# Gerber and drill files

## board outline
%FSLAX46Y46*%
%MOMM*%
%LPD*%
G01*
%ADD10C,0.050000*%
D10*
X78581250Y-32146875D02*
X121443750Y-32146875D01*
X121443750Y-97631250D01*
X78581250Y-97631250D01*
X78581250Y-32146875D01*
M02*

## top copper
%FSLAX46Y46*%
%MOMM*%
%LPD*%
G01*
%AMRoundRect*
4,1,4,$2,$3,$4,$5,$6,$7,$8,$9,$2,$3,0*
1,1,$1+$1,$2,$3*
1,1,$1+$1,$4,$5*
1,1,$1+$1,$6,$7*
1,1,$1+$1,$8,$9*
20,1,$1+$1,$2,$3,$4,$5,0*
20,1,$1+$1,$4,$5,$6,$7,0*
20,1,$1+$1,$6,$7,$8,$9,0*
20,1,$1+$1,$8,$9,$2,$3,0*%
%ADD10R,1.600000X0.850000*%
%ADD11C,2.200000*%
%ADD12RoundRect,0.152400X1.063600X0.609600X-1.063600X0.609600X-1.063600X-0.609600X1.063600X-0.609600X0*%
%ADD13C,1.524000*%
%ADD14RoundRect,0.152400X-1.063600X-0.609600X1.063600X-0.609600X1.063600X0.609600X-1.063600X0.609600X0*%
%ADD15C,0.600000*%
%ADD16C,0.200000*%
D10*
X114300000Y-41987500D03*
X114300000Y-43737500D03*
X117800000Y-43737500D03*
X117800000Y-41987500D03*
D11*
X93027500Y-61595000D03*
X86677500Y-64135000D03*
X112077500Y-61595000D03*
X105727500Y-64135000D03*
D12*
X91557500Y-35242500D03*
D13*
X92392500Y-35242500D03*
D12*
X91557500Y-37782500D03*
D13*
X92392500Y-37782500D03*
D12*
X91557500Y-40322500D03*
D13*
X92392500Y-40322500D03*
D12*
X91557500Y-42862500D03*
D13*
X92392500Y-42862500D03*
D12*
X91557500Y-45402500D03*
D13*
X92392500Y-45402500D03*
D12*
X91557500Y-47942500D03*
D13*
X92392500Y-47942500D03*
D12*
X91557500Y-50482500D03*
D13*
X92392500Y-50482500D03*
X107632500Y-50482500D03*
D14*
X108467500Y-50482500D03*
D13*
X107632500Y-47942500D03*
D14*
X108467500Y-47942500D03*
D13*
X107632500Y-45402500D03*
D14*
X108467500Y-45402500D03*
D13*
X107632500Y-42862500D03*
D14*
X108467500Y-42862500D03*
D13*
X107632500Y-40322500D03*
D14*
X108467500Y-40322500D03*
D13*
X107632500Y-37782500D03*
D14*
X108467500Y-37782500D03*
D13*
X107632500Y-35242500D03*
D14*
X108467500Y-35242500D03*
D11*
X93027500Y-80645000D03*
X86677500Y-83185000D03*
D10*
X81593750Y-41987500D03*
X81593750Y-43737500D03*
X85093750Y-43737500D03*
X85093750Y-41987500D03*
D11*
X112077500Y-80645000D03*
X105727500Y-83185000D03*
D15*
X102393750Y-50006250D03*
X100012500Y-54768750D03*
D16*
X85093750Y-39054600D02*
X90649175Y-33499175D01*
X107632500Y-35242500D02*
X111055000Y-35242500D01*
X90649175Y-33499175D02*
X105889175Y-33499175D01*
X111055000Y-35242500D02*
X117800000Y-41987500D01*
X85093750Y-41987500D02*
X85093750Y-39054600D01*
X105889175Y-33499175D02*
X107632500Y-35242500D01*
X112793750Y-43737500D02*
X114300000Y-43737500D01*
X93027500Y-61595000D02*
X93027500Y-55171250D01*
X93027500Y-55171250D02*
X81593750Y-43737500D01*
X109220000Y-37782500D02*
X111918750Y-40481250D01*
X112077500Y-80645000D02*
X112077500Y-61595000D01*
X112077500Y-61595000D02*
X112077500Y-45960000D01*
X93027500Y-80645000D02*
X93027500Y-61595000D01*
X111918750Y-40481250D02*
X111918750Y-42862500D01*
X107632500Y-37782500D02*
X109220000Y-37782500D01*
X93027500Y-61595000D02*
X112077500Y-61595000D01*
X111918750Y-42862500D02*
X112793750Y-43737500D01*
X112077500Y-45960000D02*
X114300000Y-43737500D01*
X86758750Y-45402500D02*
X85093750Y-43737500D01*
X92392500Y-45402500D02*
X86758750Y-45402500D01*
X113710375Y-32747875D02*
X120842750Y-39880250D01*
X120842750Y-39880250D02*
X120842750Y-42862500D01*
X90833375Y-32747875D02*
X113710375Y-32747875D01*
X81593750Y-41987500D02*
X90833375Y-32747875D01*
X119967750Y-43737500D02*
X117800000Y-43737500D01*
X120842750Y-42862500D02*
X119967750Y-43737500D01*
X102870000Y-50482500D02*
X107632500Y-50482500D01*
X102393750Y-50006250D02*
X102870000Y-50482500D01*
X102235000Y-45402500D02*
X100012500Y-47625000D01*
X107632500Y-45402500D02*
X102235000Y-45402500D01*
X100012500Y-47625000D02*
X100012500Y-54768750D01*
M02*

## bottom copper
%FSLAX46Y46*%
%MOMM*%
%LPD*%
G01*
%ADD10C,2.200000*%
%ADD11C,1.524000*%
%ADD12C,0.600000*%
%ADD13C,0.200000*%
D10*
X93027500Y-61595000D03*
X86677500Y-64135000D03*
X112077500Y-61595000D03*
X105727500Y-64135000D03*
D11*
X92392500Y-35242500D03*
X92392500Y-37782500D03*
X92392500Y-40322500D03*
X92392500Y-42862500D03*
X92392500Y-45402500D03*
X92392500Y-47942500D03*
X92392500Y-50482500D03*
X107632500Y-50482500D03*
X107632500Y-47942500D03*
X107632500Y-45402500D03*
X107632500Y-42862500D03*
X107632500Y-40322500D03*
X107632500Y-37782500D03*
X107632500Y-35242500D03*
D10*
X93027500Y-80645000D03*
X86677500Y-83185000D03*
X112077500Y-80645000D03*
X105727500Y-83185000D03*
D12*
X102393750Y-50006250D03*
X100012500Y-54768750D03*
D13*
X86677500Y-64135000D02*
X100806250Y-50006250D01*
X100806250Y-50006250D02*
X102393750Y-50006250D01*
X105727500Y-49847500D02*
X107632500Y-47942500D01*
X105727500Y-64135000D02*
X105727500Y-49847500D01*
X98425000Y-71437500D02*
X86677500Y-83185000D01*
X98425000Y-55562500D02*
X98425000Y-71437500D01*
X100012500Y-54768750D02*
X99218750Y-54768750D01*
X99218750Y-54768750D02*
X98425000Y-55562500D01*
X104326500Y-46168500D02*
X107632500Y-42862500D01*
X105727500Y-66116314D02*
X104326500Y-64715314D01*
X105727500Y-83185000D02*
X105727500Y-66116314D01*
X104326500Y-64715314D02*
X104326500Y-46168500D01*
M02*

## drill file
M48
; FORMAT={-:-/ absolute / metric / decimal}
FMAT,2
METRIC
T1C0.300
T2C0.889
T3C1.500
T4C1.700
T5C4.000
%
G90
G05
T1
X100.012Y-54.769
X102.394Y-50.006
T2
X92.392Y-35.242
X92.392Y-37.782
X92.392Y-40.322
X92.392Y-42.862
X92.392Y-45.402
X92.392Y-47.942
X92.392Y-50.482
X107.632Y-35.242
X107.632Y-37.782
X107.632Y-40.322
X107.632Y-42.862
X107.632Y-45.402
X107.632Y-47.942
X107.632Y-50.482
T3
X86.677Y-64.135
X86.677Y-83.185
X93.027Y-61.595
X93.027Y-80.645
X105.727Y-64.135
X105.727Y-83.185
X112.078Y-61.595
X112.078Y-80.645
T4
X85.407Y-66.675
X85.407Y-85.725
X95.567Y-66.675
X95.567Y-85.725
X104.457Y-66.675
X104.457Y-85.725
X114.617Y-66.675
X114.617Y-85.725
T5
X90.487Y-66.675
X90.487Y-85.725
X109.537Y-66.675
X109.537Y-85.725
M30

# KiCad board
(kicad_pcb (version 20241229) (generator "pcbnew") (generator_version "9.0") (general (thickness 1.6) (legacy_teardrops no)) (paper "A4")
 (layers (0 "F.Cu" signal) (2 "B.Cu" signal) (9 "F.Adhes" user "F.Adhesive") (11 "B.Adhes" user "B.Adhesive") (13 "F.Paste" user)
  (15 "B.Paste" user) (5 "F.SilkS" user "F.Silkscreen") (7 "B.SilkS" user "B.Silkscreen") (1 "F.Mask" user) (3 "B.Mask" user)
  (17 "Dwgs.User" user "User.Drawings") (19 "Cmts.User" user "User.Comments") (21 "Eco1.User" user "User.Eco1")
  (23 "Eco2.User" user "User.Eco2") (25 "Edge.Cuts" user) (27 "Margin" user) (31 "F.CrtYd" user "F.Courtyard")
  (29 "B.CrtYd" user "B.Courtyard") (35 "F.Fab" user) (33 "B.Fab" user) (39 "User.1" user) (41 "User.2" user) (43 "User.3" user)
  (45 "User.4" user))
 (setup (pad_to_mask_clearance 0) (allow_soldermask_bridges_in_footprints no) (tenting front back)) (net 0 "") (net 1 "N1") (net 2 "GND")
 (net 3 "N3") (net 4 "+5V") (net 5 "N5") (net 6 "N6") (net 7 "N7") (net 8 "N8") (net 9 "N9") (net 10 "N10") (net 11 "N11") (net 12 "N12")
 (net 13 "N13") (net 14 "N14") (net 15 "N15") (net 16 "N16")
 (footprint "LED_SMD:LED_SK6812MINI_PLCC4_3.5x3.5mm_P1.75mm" (layer "F.Cu") (at 116.05 42.8625)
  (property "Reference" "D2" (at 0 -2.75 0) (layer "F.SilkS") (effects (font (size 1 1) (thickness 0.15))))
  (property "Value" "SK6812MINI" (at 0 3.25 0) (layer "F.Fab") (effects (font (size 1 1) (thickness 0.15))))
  (pad "1" smd rect (at -1.75 -0.875) (size 1.6 0.85) (layers "F.Cu" "F.Mask" "F.Paste") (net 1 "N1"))
  (pad "2" smd rect (at -1.75 0.875) (size 1.6 0.85) (layers "F.Cu" "F.Mask" "F.Paste") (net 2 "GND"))
  (pad "3" smd rect (at 1.75 0.875) (size 1.6 0.85) (layers "F.Cu" "F.Mask" "F.Paste") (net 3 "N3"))
  (pad "4" smd rect (at 1.75 -0.875) (size 1.6 0.85) (layers "F.Cu" "F.Mask" "F.Paste") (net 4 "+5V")))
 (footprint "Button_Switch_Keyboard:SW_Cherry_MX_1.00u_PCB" (layer "F.Cu") (at 93.0275 61.595)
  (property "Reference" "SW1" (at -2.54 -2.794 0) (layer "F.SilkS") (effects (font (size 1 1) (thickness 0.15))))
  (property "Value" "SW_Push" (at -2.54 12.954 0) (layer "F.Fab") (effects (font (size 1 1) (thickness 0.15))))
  (pad "" np_thru_hole circle (at -7.62 5.08) (size 1.7 1.7) (drill 1.7) (layers "*.Cu" "*.Mask"))
  (pad "" np_thru_hole circle (at -2.54 5.08) (size 4 4) (drill 4) (layers "*.Cu" "*.Mask"))
  (pad "" np_thru_hole circle (at 2.54 5.08) (size 1.7 1.7) (drill 1.7) (layers "*.Cu" "*.Mask"))
  (pad "1" thru_hole circle (at 0 0) (size 2.2 2.2) (drill 1.5) (layers "*.Cu" "*.Mask") (remove_unused_layers no) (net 2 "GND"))
  (pad "2" thru_hole circle (at -6.35 2.54) (size 2.2 2.2) (drill 1.5) (layers "*.Cu" "*.Mask") (remove_unused_layers no) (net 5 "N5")))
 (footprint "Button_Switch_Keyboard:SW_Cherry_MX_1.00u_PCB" (layer "F.Cu") (at 112.0775 61.595)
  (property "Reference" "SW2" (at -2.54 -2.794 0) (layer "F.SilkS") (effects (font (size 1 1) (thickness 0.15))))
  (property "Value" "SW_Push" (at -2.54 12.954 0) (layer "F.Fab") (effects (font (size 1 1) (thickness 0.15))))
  (pad "" np_thru_hole circle (at -7.62 5.08) (size 1.7 1.7) (drill 1.7) (layers "*.Cu" "*.Mask"))
  (pad "" np_thru_hole circle (at -2.54 5.08) (size 4 4) (drill 4) (layers "*.Cu" "*.Mask"))
  (pad "" np_thru_hole circle (at 2.54 5.08) (size 1.7 1.7) (drill 1.7) (layers "*.Cu" "*.Mask"))
  (pad "1" thru_hole circle (at 0 0) (size 2.2 2.2) (drill 1.5) (layers "*.Cu" "*.Mask") (remove_unused_layers no) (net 2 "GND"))
  (pad "2" thru_hole circle (at -6.35 2.54) (size 2.2 2.2) (drill 1.5) (layers "*.Cu" "*.Mask") (remove_unused_layers no) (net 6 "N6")))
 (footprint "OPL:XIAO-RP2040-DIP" (layer "F.Cu") (at 100.0125 42.8625)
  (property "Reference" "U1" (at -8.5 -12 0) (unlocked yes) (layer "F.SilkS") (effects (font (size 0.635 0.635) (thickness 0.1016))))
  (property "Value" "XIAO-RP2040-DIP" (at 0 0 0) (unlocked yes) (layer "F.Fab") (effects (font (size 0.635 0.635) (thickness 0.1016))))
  (pad "1" smd roundrect (at -8.455 -7.62 180) (size 2.432 1.524) (layers "F.Cu" "F.Mask") (roundrect_rratio 0.1) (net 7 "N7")
   (thermal_bridge_angle 45))
  (pad "1" thru_hole circle (at -7.62 -7.62 180) (size 1.524 1.524) (drill 0.889) (layers "*.Cu" "*.Mask") (remove_unused_layers no)
   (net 7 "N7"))
  (pad "2" smd roundrect (at -8.455 -5.08 180) (size 2.432 1.524) (layers "F.Cu" "F.Mask") (roundrect_rratio 0.1) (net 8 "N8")
   (thermal_bridge_angle 45))
  (pad "2" thru_hole circle (at -7.62 -5.08 180) (size 1.524 1.524) (drill 0.889) (layers "*.Cu" "*.Mask") (remove_unused_layers no)
   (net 8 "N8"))
  (pad "3" smd roundrect (at -8.455 -2.54 180) (size 2.432 1.524) (layers "F.Cu" "F.Mask") (roundrect_rratio 0.1) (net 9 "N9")
   (thermal_bridge_angle 45))
  (pad "3" thru_hole circle (at -7.62 -2.54 180) (size 1.524 1.524) (drill 0.889) (layers "*.Cu" "*.Mask") (remove_unused_layers no)
   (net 9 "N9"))
  (pad "4" smd roundrect (at -8.455 0 180) (size 2.432 1.524) (layers "F.Cu" "F.Mask") (roundrect_rratio 0.1) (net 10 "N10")
   (thermal_bridge_angle 45))
  (pad "4" thru_hole circle (at -7.62 0 180) (size 1.524 1.524) (drill 0.889) (layers "*.Cu" "*.Mask") (remove_unused_layers no)
   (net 10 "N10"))
  (pad "5" smd roundrect (at -8.455 2.54 180) (size 2.432 1.524) (layers "F.Cu" "F.Mask") (roundrect_rratio 0.1) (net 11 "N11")
   (thermal_bridge_angle 45))
  (pad "5" thru_hole circle (at -7.62 2.54 180) (size 1.524 1.524) (drill 0.889) (layers "*.Cu" "*.Mask") (remove_unused_layers no)
   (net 11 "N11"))
  (pad "6" smd roundrect (at -8.455 5.08 180) (size 2.432 1.524) (layers "F.Cu" "F.Mask") (roundrect_rratio 0.1) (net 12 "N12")
   (thermal_bridge_angle 45))
  (pad "6" thru_hole circle (at -7.62 5.08 180) (size 1.524 1.524) (drill 0.889) (layers "*.Cu" "*.Mask") (remove_unused_layers no)
   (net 12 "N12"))
  (pad "7" smd roundrect (at -8.455 7.62 180) (size 2.432 1.524) (layers "F.Cu" "F.Mask") (roundrect_rratio 0.1) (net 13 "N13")
   (thermal_bridge_angle 45))
  (pad "7" thru_hole circle (at -7.62 7.62 180) (size 1.524 1.524) (drill 0.889) (layers "*.Cu" "*.Mask") (remove_unused_layers no)
   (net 13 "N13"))
  (pad "8" thru_hole circle (at 7.62 7.62) (size 1.524 1.524) (drill 0.889) (layers "*.Cu" "*.Mask") (remove_unused_layers no) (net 5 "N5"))
  (pad "8" smd roundrect (at 8.455 7.62) (size 2.432 1.524) (layers "F.Cu" "F.Mask") (roundrect_rratio 0.1) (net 5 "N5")
   (thermal_bridge_angle 45))
  (pad "9" thru_hole circle (at 7.62 5.08) (size 1.524 1.524) (drill 0.889) (layers "*.Cu" "*.Mask") (remove_unused_layers no) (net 6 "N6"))
  (pad "9" smd roundrect (at 8.455 5.08) (size 2.432 1.524) (layers "F.Cu" "F.Mask") (roundrect_rratio 0.1) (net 6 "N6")
   (thermal_bridge_angle 45))
  (pad "10" thru_hole circle (at 7.62 2.54) (size 1.524 1.524) (drill 0.889) (layers "*.Cu" "*.Mask") (remove_unused_layers no)
   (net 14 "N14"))
  (pad "10" smd roundrect (at 8.455 2.54) (size 2.432 1.524) (layers "F.Cu" "F.Mask") (roundrect_rratio 0.1) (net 14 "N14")
   (thermal_bridge_angle 45))
  (pad "11" thru_hole circle (at 7.62 0) (size 1.524 1.524) (drill 0.889) (layers "*.Cu" "*.Mask") (remove_unused_layers no) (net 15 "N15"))
  (pad "11" smd roundrect (at 8.455 0) (size 2.432 1.524) (layers "F.Cu" "F.Mask") (roundrect_rratio 0.1) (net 15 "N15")
   (thermal_bridge_angle 45))
  (pad "12" thru_hole circle (at 7.62 -2.54) (size 1.524 1.524) (drill 0.889) (layers "*.Cu" "*.Mask") (remove_unused_layers no)
   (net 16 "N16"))
  (pad "12" smd roundrect (at 8.455 -2.54) (size 2.432 1.524) (layers "F.Cu" "F.Mask") (roundrect_rratio 0.1) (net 16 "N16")
   (thermal_bridge_angle 45))
  (pad "13" thru_hole circle (at 7.62 -5.08) (size 1.524 1.524) (drill 0.889) (layers "*.Cu" "*.Mask") (remove_unused_layers no)
   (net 2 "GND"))
  (pad "13" smd roundrect (at 8.455 -5.08) (size 2.432 1.524) (layers "F.Cu" "F.Mask") (roundrect_rratio 0.1) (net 2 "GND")
   (thermal_bridge_angle 45))
  (pad "14" thru_hole circle (at 7.62 -7.62) (size 1.524 1.524) (drill 0.889) (layers "*.Cu" "*.Mask") (remove_unused_layers no)
   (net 4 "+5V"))
  (pad "14" smd roundrect (at 8.455 -7.62) (size 2.432 1.524) (layers "F.Cu" "F.Mask") (roundrect_rratio 0.1) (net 4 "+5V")
   (thermal_bridge_angle 45)))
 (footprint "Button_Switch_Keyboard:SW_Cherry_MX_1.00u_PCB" (layer "F.Cu") (at 93.0275 80.645)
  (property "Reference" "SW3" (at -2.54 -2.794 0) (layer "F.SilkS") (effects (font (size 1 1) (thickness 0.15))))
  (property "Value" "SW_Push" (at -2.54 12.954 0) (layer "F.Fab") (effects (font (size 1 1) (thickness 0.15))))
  (pad "" np_thru_hole circle (at -7.62 5.08) (size 1.7 1.7) (drill 1.7) (layers "*.Cu" "*.Mask"))
  (pad "" np_thru_hole circle (at -2.54 5.08) (size 4 4) (drill 4) (layers "*.Cu" "*.Mask"))
  (pad "" np_thru_hole circle (at 2.54 5.08) (size 1.7 1.7) (drill 1.7) (layers "*.Cu" "*.Mask"))
  (pad "1" thru_hole circle (at 0 0) (size 2.2 2.2) (drill 1.5) (layers "*.Cu" "*.Mask") (remove_unused_layers no) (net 2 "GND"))
  (pad "2" thru_hole circle (at -6.35 2.54) (size 2.2 2.2) (drill 1.5) (layers "*.Cu" "*.Mask") (remove_unused_layers no) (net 14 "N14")))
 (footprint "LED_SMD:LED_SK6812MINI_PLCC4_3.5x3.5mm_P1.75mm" (layer "F.Cu") (at 83.34375 42.8625)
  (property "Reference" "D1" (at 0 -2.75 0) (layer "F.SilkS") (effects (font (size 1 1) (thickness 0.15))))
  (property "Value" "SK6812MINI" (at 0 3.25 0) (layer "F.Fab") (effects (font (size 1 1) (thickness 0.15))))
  (pad "1" smd rect (at -1.75 -0.875) (size 1.6 0.85) (layers "F.Cu" "F.Mask" "F.Paste") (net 3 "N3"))
  (pad "2" smd rect (at -1.75 0.875) (size 1.6 0.85) (layers "F.Cu" "F.Mask" "F.Paste") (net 2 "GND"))
  (pad "3" smd rect (at 1.75 0.875) (size 1.6 0.85) (layers "F.Cu" "F.Mask" "F.Paste") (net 11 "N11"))
  (pad "4" smd rect (at 1.75 -0.875) (size 1.6 0.85) (layers "F.Cu" "F.Mask" "F.Paste") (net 4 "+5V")))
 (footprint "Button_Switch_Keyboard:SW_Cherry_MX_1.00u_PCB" (layer "F.Cu") (at 112.0775 80.645)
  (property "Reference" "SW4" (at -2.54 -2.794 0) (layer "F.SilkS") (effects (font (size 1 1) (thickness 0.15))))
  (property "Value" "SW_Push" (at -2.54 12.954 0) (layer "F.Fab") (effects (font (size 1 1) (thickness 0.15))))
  (pad "" np_thru_hole circle (at -7.62 5.08) (size 1.7 1.7) (drill 1.7) (layers "*.Cu" "*.Mask"))
  (pad "" np_thru_hole circle (at -2.54 5.08) (size 4 4) (drill 4) (layers "*.Cu" "*.Mask"))
  (pad "" np_thru_hole circle (at 2.54 5.08) (size 1.7 1.7) (drill 1.7) (layers "*.Cu" "*.Mask"))
  (pad "1" thru_hole circle (at 0 0) (size 2.2 2.2) (drill 1.5) (layers "*.Cu" "*.Mask") (remove_unused_layers no) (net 2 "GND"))
  (pad "2" thru_hole circle (at -6.35 2.54) (size 2.2 2.2) (drill 1.5) (layers "*.Cu" "*.Mask") (remove_unused_layers no) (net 15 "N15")))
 (gr_rect (start 78.58125 32.146875) (end 121.44375 97.63125) (stroke (width 0.05) (type solid)) (fill no) (layer "Edge.Cuts"))
 (segment (start 85.09375 39.0546) (end 90.649175 33.499175) (width 0.2) (layer "F.Cu") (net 4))
 (segment (start 107.6325 35.2425) (end 111.055 35.2425) (width 0.2) (layer "F.Cu") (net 4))
 (segment (start 90.649175 33.499175) (end 105.889175 33.499175) (width 0.2) (layer "F.Cu") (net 4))
 (segment (start 111.055 35.2425) (end 117.8 41.9875) (width 0.2) (layer "F.Cu") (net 4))
 (segment (start 85.09375 41.9875) (end 85.09375 39.0546) (width 0.2) (layer "F.Cu") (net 4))
 (segment (start 105.889175 33.499175) (end 107.6325 35.2425) (width 0.2) (layer "F.Cu") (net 4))
 (segment (start 112.79375 43.7375) (end 114.3 43.7375) (width 0.2) (layer "F.Cu") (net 2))
 (segment (start 93.0275 61.595) (end 93.0275 55.17125) (width 0.2) (layer "F.Cu") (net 2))
 (segment (start 93.0275 55.17125) (end 81.59375 43.7375) (width 0.2) (layer "F.Cu") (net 2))
 (segment (start 109.22 37.7825) (end 111.91875 40.48125) (width 0.2) (layer "F.Cu") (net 2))
 (segment (start 112.0775 80.645) (end 112.0775 61.595) (width 0.2) (layer "F.Cu") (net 2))
 (segment (start 112.0775 61.595) (end 112.0775 45.96) (width 0.2) (layer "F.Cu") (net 2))
 (segment (start 93.0275 80.645) (end 93.0275 61.595) (width 0.2) (layer "F.Cu") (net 2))
 (segment (start 111.91875 40.48125) (end 111.91875 42.8625) (width 0.2) (layer "F.Cu") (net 2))
 (segment (start 107.6325 37.7825) (end 109.22 37.7825) (width 0.2) (layer "F.Cu") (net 2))
 (segment (start 93.0275 61.595) (end 112.0775 61.595) (width 0.2) (layer "F.Cu") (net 2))
 (segment (start 111.91875 42.8625) (end 112.79375 43.7375) (width 0.2) (layer "F.Cu") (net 2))
 (segment (start 112.0775 45.96) (end 114.3 43.7375) (width 0.2) (layer "F.Cu") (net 2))
 (segment (start 86.75875 45.4025) (end 85.09375 43.7375) (width 0.2) (layer "F.Cu") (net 11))
 (segment (start 92.3925 45.4025) (end 86.75875 45.4025) (width 0.2) (layer "F.Cu") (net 11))
 (segment (start 113.710375 32.747875) (end 120.84275 39.88025) (width 0.2) (layer "F.Cu") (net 3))
 (segment (start 120.84275 39.88025) (end 120.84275 42.8625) (width 0.2) (layer "F.Cu") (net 3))
 (segment (start 90.833375 32.747875) (end 113.710375 32.747875) (width 0.2) (layer "F.Cu") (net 3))
 (segment (start 81.59375 41.9875) (end 90.833375 32.747875) (width 0.2) (layer "F.Cu") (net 3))
 (segment (start 119.96775 43.7375) (end 117.8 43.7375) (width 0.2) (layer "F.Cu") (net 3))
 (segment (start 120.84275 42.8625) (end 119.96775 43.7375) (width 0.2) (layer "F.Cu") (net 3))
 (segment (start 102.87 50.4825) (end 107.6325 50.4825) (width 0.2) (layer "F.Cu") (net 5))
 (segment (start 102.39375 50.00625) (end 102.87 50.4825) (width 0.2) (layer "F.Cu") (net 5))
 (via (at 102.39375 50.00625) (size 0.6) (drill 0.3) (layers "F.Cu" "B.Cu") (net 5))
 (segment (start 86.6775 64.135) (end 100.80625 50.00625) (width 0.2) (layer "B.Cu") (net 5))
 (segment (start 100.80625 50.00625) (end 102.39375 50.00625) (width 0.2) (layer "B.Cu") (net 5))
 (segment (start 105.7275 49.8475) (end 107.6325 47.9425) (width 0.2) (layer "B.Cu") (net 6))
 (segment (start 105.7275 64.135) (end 105.7275 49.8475) (width 0.2) (layer "B.Cu") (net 6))
 (segment (start 102.235 45.4025) (end 100.0125 47.625) (width 0.2) (layer "F.Cu") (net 14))
 (segment (start 107.6325 45.4025) (end 102.235 45.4025) (width 0.2) (layer "F.Cu") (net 14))
 (segment (start 100.0125 47.625) (end 100.0125 54.76875) (width 0.2) (layer "F.Cu") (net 14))
 (via (at 100.0125 54.76875) (size 0.6) (drill 0.3) (layers "F.Cu" "B.Cu") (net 14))
 (segment (start 98.425 71.4375) (end 86.6775 83.185) (width 0.2) (layer "B.Cu") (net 14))
 (segment (start 98.425 55.5625) (end 98.425 71.4375) (width 0.2) (layer "B.Cu") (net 14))
 (segment (start 100.0125 54.76875) (end 99.21875 54.76875) (width 0.2) (layer "B.Cu") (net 14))
 (segment (start 99.21875 54.76875) (end 98.425 55.5625) (width 0.2) (layer "B.Cu") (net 14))
 (segment (start 104.3265 46.1685) (end 107.6325 42.8625) (width 0.2) (layer "B.Cu") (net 15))
 (segment (start 105.7275 66.116314) (end 104.3265 64.715314) (width 0.2) (layer "B.Cu") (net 15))
 (segment (start 105.7275 83.185) (end 105.7275 66.116314) (width 0.2) (layer "B.Cu") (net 15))
 (segment (start 104.3265 64.715314) (end 104.3265 46.1685) (width 0.2) (layer "B.Cu") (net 15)))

